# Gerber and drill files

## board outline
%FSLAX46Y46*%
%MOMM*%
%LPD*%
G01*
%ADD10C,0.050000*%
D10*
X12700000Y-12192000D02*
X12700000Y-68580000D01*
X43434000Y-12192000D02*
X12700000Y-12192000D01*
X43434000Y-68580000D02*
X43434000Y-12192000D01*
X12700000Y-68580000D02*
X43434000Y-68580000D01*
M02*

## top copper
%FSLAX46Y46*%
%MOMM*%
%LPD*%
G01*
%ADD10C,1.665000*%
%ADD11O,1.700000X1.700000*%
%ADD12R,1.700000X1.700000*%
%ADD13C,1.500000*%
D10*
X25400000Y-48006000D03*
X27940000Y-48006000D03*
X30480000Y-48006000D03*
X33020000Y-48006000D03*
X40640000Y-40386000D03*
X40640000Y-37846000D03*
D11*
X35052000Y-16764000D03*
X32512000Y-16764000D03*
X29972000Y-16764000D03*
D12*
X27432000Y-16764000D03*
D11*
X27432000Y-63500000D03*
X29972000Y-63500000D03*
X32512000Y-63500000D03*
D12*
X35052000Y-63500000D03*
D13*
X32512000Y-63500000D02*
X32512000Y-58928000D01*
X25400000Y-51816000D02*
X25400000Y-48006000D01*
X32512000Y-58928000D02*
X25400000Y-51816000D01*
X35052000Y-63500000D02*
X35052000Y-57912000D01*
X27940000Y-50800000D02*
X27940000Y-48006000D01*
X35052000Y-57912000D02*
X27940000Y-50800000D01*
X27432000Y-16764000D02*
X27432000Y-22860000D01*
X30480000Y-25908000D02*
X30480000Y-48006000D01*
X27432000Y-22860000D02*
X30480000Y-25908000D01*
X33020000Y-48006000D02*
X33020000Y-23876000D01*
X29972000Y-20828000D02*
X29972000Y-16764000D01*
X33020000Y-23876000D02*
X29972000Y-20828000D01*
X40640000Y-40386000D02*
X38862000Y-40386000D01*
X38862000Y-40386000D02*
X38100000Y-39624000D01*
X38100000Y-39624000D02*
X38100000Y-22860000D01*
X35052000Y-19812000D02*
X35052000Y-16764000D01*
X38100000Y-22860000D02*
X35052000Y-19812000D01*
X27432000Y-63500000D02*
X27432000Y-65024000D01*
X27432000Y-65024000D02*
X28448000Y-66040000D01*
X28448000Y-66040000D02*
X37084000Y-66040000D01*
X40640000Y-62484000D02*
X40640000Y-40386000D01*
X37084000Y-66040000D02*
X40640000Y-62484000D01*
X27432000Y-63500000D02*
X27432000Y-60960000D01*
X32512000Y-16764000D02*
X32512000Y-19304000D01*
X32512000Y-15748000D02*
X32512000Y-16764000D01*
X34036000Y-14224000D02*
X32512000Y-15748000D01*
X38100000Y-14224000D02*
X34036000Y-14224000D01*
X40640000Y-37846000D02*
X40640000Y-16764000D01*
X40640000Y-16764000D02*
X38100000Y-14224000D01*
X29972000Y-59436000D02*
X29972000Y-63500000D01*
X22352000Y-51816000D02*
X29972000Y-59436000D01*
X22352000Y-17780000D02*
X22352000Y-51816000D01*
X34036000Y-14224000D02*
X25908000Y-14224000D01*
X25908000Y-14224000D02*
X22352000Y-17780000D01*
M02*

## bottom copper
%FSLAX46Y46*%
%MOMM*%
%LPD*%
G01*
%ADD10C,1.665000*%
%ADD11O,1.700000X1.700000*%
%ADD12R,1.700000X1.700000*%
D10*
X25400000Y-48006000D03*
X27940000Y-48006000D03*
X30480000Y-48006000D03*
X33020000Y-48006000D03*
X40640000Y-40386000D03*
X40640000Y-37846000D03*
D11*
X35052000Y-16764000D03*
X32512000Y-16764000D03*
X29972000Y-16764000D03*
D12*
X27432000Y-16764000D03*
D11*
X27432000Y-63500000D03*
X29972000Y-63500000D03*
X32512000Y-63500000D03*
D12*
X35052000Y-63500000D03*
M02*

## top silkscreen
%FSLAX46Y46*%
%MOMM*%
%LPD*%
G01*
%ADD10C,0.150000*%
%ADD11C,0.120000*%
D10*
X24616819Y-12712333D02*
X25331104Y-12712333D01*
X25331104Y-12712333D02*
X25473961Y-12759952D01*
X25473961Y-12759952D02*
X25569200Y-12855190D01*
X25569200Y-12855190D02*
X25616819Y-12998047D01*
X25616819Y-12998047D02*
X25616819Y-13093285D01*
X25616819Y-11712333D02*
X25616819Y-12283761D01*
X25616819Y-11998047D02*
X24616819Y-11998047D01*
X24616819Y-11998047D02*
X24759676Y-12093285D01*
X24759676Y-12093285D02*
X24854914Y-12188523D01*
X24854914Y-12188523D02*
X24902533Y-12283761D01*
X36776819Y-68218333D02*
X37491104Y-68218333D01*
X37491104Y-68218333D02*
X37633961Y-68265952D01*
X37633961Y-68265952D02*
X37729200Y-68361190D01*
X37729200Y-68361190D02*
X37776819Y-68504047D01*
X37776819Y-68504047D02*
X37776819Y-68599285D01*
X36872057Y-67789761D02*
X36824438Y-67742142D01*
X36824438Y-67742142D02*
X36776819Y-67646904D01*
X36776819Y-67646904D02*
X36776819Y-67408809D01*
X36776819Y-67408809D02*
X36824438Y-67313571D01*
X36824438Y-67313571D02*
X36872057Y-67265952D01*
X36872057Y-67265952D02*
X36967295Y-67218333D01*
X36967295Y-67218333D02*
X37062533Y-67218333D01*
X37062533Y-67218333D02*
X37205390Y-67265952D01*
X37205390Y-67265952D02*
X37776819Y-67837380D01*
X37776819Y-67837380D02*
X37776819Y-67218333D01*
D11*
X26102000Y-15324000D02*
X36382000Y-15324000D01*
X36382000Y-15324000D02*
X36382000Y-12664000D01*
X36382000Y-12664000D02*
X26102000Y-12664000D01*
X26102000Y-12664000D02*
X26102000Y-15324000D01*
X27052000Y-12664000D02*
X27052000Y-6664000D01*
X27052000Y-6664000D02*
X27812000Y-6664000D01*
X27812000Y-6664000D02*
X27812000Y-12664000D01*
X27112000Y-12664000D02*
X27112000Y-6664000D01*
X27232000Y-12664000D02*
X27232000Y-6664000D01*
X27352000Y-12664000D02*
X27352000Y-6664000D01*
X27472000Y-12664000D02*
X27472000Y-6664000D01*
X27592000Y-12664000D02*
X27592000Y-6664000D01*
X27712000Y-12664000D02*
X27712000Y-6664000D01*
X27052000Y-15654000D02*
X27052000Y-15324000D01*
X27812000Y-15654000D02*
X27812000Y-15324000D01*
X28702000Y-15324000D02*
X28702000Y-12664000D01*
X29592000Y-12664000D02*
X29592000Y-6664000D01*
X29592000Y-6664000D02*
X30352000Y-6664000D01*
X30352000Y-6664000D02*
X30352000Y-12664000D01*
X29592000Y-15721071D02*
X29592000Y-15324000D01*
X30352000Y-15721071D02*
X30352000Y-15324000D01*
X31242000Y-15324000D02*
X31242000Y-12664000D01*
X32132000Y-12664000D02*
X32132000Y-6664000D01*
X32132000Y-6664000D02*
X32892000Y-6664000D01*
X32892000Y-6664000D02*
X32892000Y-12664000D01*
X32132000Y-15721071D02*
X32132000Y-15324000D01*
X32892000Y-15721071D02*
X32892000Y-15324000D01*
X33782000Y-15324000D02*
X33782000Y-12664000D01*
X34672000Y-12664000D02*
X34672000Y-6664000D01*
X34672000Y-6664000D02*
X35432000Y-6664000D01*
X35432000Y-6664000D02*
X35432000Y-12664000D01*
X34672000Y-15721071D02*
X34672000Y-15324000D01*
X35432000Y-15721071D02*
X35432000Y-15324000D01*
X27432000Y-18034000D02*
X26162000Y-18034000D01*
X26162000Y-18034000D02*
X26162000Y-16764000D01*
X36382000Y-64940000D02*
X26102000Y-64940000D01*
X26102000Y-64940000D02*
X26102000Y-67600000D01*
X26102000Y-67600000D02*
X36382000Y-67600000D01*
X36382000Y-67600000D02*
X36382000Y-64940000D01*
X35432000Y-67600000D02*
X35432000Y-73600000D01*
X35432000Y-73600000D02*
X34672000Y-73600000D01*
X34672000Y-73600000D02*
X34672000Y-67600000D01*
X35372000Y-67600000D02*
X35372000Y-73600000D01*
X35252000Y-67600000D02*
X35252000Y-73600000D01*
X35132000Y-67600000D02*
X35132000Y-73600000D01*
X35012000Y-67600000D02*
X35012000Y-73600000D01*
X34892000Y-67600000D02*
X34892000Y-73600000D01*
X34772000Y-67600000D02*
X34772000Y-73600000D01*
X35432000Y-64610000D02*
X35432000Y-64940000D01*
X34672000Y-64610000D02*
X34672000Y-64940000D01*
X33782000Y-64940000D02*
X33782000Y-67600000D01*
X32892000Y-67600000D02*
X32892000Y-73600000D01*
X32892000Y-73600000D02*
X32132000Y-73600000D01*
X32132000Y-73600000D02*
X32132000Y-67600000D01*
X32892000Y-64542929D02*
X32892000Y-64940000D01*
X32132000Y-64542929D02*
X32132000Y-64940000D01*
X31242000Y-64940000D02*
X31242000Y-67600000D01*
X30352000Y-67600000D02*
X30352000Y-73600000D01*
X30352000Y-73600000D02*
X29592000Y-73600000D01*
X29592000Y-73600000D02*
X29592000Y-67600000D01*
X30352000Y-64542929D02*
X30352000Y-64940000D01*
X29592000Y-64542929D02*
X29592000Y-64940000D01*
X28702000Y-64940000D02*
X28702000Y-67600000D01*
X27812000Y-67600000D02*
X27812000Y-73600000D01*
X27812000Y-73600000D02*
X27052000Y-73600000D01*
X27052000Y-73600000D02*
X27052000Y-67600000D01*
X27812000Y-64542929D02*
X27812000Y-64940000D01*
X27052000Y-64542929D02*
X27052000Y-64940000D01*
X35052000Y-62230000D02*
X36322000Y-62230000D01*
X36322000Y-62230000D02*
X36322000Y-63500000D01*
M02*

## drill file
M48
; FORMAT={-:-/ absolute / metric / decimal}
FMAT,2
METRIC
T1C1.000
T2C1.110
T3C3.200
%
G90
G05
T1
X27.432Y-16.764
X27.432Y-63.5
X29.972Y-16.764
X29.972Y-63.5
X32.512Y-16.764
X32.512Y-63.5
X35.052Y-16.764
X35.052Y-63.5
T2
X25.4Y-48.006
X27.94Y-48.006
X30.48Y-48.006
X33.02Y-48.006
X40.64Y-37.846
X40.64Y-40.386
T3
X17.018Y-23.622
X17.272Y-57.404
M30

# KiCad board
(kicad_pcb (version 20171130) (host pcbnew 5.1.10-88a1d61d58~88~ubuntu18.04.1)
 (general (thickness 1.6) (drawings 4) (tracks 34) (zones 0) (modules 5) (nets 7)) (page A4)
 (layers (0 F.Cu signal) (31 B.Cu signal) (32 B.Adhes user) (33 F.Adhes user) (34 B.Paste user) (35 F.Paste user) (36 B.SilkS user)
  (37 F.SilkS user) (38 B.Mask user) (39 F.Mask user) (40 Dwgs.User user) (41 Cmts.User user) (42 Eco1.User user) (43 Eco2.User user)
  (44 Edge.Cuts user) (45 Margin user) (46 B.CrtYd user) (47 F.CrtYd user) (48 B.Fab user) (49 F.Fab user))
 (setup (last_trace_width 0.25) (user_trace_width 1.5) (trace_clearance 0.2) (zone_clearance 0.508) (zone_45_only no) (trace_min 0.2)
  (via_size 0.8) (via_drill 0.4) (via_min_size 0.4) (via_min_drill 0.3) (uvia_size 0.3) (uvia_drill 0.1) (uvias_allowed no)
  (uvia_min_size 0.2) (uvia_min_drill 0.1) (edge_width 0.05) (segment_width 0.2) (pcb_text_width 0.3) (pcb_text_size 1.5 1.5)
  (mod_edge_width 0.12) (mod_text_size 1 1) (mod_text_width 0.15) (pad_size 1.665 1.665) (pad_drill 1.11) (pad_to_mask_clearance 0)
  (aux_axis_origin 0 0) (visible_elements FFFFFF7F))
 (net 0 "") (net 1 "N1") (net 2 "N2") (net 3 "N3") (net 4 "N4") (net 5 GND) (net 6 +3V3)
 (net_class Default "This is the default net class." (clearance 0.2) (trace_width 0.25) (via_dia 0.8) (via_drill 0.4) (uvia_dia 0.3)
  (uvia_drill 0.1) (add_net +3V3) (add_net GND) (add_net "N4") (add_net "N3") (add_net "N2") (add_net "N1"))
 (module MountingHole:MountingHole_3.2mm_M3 (layer B.Cu) (at 17.018 23.622)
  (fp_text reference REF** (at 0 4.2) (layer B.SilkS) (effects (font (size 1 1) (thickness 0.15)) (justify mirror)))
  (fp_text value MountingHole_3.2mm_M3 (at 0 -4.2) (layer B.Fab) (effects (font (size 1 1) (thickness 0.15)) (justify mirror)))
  (pad 1 np_thru_hole circle (at 0 0) (size 3.2 3.2) (drill 3.2) (layers *.Cu *.Mask)))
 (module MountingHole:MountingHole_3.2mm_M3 (layer B.Cu) (at 17.272 57.404)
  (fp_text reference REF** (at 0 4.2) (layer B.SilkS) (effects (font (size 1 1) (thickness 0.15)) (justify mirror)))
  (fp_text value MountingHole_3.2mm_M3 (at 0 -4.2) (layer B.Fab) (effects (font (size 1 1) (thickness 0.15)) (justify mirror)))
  (pad 1 np_thru_hole circle (at 0 0) (size 3.2 3.2) (drill 3.2) (layers *.Cu *.Mask)))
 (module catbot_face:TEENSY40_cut (layer B.Cu) (at 7.62 32.766)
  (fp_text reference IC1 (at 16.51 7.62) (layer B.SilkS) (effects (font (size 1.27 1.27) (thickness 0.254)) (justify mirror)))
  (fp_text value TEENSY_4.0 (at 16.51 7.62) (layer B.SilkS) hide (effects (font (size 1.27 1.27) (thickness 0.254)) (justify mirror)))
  (pad 26 thru_hole circle (at 17.78 15.24 270) (size 1.665 1.665) (drill 1.11) (layers *.Cu *.Mask B.SilkS) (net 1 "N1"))
  (pad 25 thru_hole circle (at 20.32 15.24 270) (size 1.665 1.665) (drill 1.11) (layers *.Cu *.Mask B.SilkS) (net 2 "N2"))
  (pad 24 thru_hole circle (at 22.86 15.24 270) (size 1.665 1.665) (drill 1.11) (layers *.Cu *.Mask B.SilkS) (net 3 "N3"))
  (pad 23 thru_hole circle (at 25.4 15.24 270) (size 1.665 1.665) (drill 1.11) (layers *.Cu *.Mask B.SilkS) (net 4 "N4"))
  (pad 17 thru_hole circle (at 33.02 7.62 270) (size 1.665 1.665) (drill 1.11) (layers *.Cu *.Mask B.SilkS) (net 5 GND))
  (pad 16 thru_hole circle (at 33.02 5.08 270) (size 1.665 1.665) (drill 1.11) (layers *.Cu *.Mask B.SilkS) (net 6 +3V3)))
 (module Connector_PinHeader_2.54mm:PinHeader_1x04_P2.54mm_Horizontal (layer F.Cu) (at 27.432 16.764 90)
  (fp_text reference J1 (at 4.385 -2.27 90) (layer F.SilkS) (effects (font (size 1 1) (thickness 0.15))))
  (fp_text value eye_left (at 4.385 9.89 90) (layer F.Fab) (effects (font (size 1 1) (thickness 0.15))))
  (fp_line (start 1.44 -1.33) (end 1.44 8.95) (layer F.SilkS) (width 0.12))
  (fp_line (start 1.44 8.95) (end 4.1 8.95) (layer F.SilkS) (width 0.12))
  (fp_line (start 4.1 8.95) (end 4.1 -1.33) (layer F.SilkS) (width 0.12))
  (fp_line (start 4.1 -1.33) (end 1.44 -1.33) (layer F.SilkS) (width 0.12))
  (fp_line (start 4.1 -0.38) (end 10.1 -0.38) (layer F.SilkS) (width 0.12))
  (fp_line (start 10.1 -0.38) (end 10.1 0.38) (layer F.SilkS) (width 0.12))
  (fp_line (start 10.1 0.38) (end 4.1 0.38) (layer F.SilkS) (width 0.12))
  (fp_line (start 4.1 -0.32) (end 10.1 -0.32) (layer F.SilkS) (width 0.12))
  (fp_line (start 4.1 -0.2) (end 10.1 -0.2) (layer F.SilkS) (width 0.12))
  (fp_line (start 4.1 -0.08) (end 10.1 -0.08) (layer F.SilkS) (width 0.12))
  (fp_line (start 4.1 0.04) (end 10.1 0.04) (layer F.SilkS) (width 0.12))
  (fp_line (start 4.1 0.16) (end 10.1 0.16) (layer F.SilkS) (width 0.12))
  (fp_line (start 4.1 0.28) (end 10.1 0.28) (layer F.SilkS) (width 0.12))
  (fp_line (start 1.11 -0.38) (end 1.44 -0.38) (layer F.SilkS) (width 0.12))
  (fp_line (start 1.11 0.38) (end 1.44 0.38) (layer F.SilkS) (width 0.12))
  (fp_line (start 1.44 1.27) (end 4.1 1.27) (layer F.SilkS) (width 0.12))
  (fp_line (start 4.1 2.16) (end 10.1 2.16) (layer F.SilkS) (width 0.12))
  (fp_line (start 10.1 2.16) (end 10.1 2.92) (layer F.SilkS) (width 0.12))
  (fp_line (start 10.1 2.92) (end 4.1 2.92) (layer F.SilkS) (width 0.12))
  (fp_line (start 1.042929 2.16) (end 1.44 2.16) (layer F.SilkS) (width 0.12))
  (fp_line (start 1.042929 2.92) (end 1.44 2.92) (layer F.SilkS) (width 0.12))
  (fp_line (start 1.44 3.81) (end 4.1 3.81) (layer F.SilkS) (width 0.12))
  (fp_line (start 4.1 4.7) (end 10.1 4.7) (layer F.SilkS) (width 0.12))
  (fp_line (start 10.1 4.7) (end 10.1 5.46) (layer F.SilkS) (width 0.12))
  (fp_line (start 10.1 5.46) (end 4.1 5.46) (layer F.SilkS) (width 0.12))
  (fp_line (start 1.042929 4.7) (end 1.44 4.7) (layer F.SilkS) (width 0.12))
  (fp_line (start 1.042929 5.46) (end 1.44 5.46) (layer F.SilkS) (width 0.12))
  (fp_line (start 1.44 6.35) (end 4.1 6.35) (layer F.SilkS) (width 0.12))
  (fp_line (start 4.1 7.24) (end 10.1 7.24) (layer F.SilkS) (width 0.12))
  (fp_line (start 10.1 7.24) (end 10.1 8) (layer F.SilkS) (width 0.12))
  (fp_line (start 10.1 8) (end 4.1 8) (layer F.SilkS) (width 0.12))
  (fp_line (start 1.042929 7.24) (end 1.44 7.24) (layer F.SilkS) (width 0.12))
  (fp_line (start 1.042929 8) (end 1.44 8) (layer F.SilkS) (width 0.12))
  (fp_line (start -1.27 0) (end -1.27 -1.27) (layer F.SilkS) (width 0.12))
  (fp_line (start -1.27 -1.27) (end 0 -1.27) (layer F.SilkS) (width 0.12))
  (pad 4 thru_hole oval (at 0 7.62 90) (size 1.7 1.7) (drill 1) (layers *.Cu *.Mask) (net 5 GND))
  (pad 3 thru_hole oval (at 0 5.08 90) (size 1.7 1.7) (drill 1) (layers *.Cu *.Mask) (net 6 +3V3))
  (pad 2 thru_hole oval (at 0 2.54 90) (size 1.7 1.7) (drill 1) (layers *.Cu *.Mask) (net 4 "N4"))
  (pad 1 thru_hole rect (at 0 0 90) (size 1.7 1.7) (drill 1) (layers *.Cu *.Mask) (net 3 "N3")))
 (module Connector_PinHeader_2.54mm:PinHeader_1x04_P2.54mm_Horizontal (layer F.Cu) (at 35.052 63.5 270)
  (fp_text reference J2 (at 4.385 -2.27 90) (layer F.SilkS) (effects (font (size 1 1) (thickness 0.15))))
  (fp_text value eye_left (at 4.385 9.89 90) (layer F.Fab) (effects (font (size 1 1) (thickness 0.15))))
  (fp_line (start 1.44 -1.33) (end 1.44 8.95) (layer F.SilkS) (width 0.12))
  (fp_line (start 1.44 8.95) (end 4.1 8.95) (layer F.SilkS) (width 0.12))
  (fp_line (start 4.1 8.95) (end 4.1 -1.33) (layer F.SilkS) (width 0.12))
  (fp_line (start 4.1 -1.33) (end 1.44 -1.33) (layer F.SilkS) (width 0.12))
  (fp_line (start 4.1 -0.38) (end 10.1 -0.38) (layer F.SilkS) (width 0.12))
  (fp_line (start 10.1 -0.38) (end 10.1 0.38) (layer F.SilkS) (width 0.12))
  (fp_line (start 10.1 0.38) (end 4.1 0.38) (layer F.SilkS) (width 0.12))
  (fp_line (start 4.1 -0.32) (end 10.1 -0.32) (layer F.SilkS) (width 0.12))
  (fp_line (start 4.1 -0.2) (end 10.1 -0.2) (layer F.SilkS) (width 0.12))
  (fp_line (start 4.1 -0.08) (end 10.1 -0.08) (layer F.SilkS) (width 0.12))
  (fp_line (start 4.1 0.04) (end 10.1 0.04) (layer F.SilkS) (width 0.12))
  (fp_line (start 4.1 0.16) (end 10.1 0.16) (layer F.SilkS) (width 0.12))
  (fp_line (start 4.1 0.28) (end 10.1 0.28) (layer F.SilkS) (width 0.12))
  (fp_line (start 1.11 -0.38) (end 1.44 -0.38) (layer F.SilkS) (width 0.12))
  (fp_line (start 1.11 0.38) (end 1.44 0.38) (layer F.SilkS) (width 0.12))
  (fp_line (start 1.44 1.27) (end 4.1 1.27) (layer F.SilkS) (width 0.12))
  (fp_line (start 4.1 2.16) (end 10.1 2.16) (layer F.SilkS) (width 0.12))
  (fp_line (start 10.1 2.16) (end 10.1 2.92) (layer F.SilkS) (width 0.12))
  (fp_line (start 10.1 2.92) (end 4.1 2.92) (layer F.SilkS) (width 0.12))
  (fp_line (start 1.042929 2.16) (end 1.44 2.16) (layer F.SilkS) (width 0.12))
  (fp_line (start 1.042929 2.92) (end 1.44 2.92) (layer F.SilkS) (width 0.12))
  (fp_line (start 1.44 3.81) (end 4.1 3.81) (layer F.SilkS) (width 0.12))
  (fp_line (start 4.1 4.7) (end 10.1 4.7) (layer F.SilkS) (width 0.12))
  (fp_line (start 10.1 4.7) (end 10.1 5.46) (layer F.SilkS) (width 0.12))
  (fp_line (start 10.1 5.46) (end 4.1 5.46) (layer F.SilkS) (width 0.12))
  (fp_line (start 1.042929 4.7) (end 1.44 4.7) (layer F.SilkS) (width 0.12))
  (fp_line (start 1.042929 5.46) (end 1.44 5.46) (layer F.SilkS) (width 0.12))
  (fp_line (start 1.44 6.35) (end 4.1 6.35) (layer F.SilkS) (width 0.12))
  (fp_line (start 4.1 7.24) (end 10.1 7.24) (layer F.SilkS) (width 0.12))
  (fp_line (start 10.1 7.24) (end 10.1 8) (layer F.SilkS) (width 0.12))
  (fp_line (start 10.1 8) (end 4.1 8) (layer F.SilkS) (width 0.12))
  (fp_line (start 1.042929 7.24) (end 1.44 7.24) (layer F.SilkS) (width 0.12))
  (fp_line (start 1.042929 8) (end 1.44 8) (layer F.SilkS) (width 0.12))
  (fp_line (start -1.27 0) (end -1.27 -1.27) (layer F.SilkS) (width 0.12))
  (fp_line (start -1.27 -1.27) (end 0 -1.27) (layer F.SilkS) (width 0.12))
  (pad 4 thru_hole oval (at 0 7.62 270) (size 1.7 1.7) (drill 1) (layers *.Cu *.Mask) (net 5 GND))
  (pad 3 thru_hole oval (at 0 5.08 270) (size 1.7 1.7) (drill 1) (layers *.Cu *.Mask) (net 6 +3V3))
  (pad 2 thru_hole oval (at 0 2.54 270) (size 1.7 1.7) (drill 1) (layers *.Cu *.Mask) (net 1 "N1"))
  (pad 1 thru_hole rect (at 0 0 270) (size 1.7 1.7) (drill 1) (layers *.Cu *.Mask) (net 2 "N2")))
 (gr_line (start 12.7 12.192) (end 12.7 68.58) (layer Edge.Cuts) (width 0.05))
 (gr_line (start 43.434 12.192) (end 12.7 12.192) (layer Edge.Cuts) (width 0.05))
 (gr_line (start 43.434 68.58) (end 43.434 12.192) (layer Edge.Cuts) (width 0.05))
 (gr_line (start 12.7 68.58) (end 43.434 68.58) (layer Edge.Cuts) (width 0.05))
 (segment (start 32.512 63.5) (end 32.512 58.928) (width 1.5) (layer F.Cu) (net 1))
 (segment (start 25.4 51.816) (end 25.4 48.006) (width 1.5) (layer F.Cu) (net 1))
 (segment (start 32.512 58.928) (end 25.4 51.816) (width 1.5) (layer F.Cu) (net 1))
 (segment (start 35.052 63.5) (end 35.052 57.912) (width 1.5) (layer F.Cu) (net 2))
 (segment (start 27.94 50.8) (end 27.94 48.006) (width 1.5) (layer F.Cu) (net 2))
 (segment (start 35.052 57.912) (end 27.94 50.8) (width 1.5) (layer F.Cu) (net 2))
 (segment (start 27.432 16.764) (end 27.432 22.86) (width 1.5) (layer F.Cu) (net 3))
 (segment (start 30.48 25.908) (end 30.48 48.006) (width 1.5) (layer F.Cu) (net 3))
 (segment (start 27.432 22.86) (end 30.48 25.908) (width 1.5) (layer F.Cu) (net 3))
 (segment (start 33.02 48.006) (end 33.02 23.876) (width 1.5) (layer F.Cu) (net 4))
 (segment (start 29.972 20.828) (end 29.972 16.764) (width 1.5) (layer F.Cu) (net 4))
 (segment (start 33.02 23.876) (end 29.972 20.828) (width 1.5) (layer F.Cu) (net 4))
 (segment (start 40.64 40.386) (end 38.862 40.386) (width 1.5) (layer F.Cu) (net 5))
 (segment (start 38.862 40.386) (end 38.1 39.624) (width 1.5) (layer F.Cu) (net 5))
 (segment (start 38.1 39.624) (end 38.1 22.86) (width 1.5) (layer F.Cu) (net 5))
 (segment (start 35.052 19.812) (end 35.052 16.764) (width 1.5) (layer F.Cu) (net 5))
 (segment (start 38.1 22.86) (end 35.052 19.812) (width 1.5) (layer F.Cu) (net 5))
 (segment (start 27.432 63.5) (end 27.432 65.024) (width 1.5) (layer F.Cu) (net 5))
 (segment (start 27.432 65.024) (end 28.448 66.04) (width 1.5) (layer F.Cu) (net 5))
 (segment (start 28.448 66.04) (end 37.084 66.04) (width 1.5) (layer F.Cu) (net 5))
 (segment (start 40.64 62.484) (end 40.64 40.386) (width 1.5) (layer F.Cu) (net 5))
 (segment (start 37.084 66.04) (end 40.64 62.484) (width 1.5) (layer F.Cu) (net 5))
 (segment (start 27.432 63.5) (end 27.432 60.96) (width 1.5) (layer F.Cu) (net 5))
 (segment (start 32.512 16.764) (end 32.512 19.304) (width 1.5) (layer F.Cu) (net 6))
 (segment (start 32.512 15.748) (end 32.512 16.764) (width 1.5) (layer F.Cu) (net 6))
 (segment (start 34.036 14.224) (end 32.512 15.748) (width 1.5) (layer F.Cu) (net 6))
 (segment (start 38.1 14.224) (end 34.036 14.224) (width 1.5) (layer F.Cu) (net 6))
 (segment (start 40.64 37.846) (end 40.64 16.764) (width 1.5) (layer F.Cu) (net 6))
 (segment (start 40.64 16.764) (end 38.1 14.224) (width 1.5) (layer F.Cu) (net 6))
 (segment (start 29.972 59.436) (end 29.972 63.5) (width 1.5) (layer F.Cu) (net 6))
 (segment (start 22.352 51.816) (end 29.972 59.436) (width 1.5) (layer F.Cu) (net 6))
 (segment (start 22.352 17.78) (end 22.352 51.816) (width 1.5) (layer F.Cu) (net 6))
 (segment (start 34.036 14.224) (end 25.908 14.224) (width 1.5) (layer F.Cu) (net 6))
 (segment (start 25.908 14.224) (end 22.352 17.78) (width 1.5) (layer F.Cu) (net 6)))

